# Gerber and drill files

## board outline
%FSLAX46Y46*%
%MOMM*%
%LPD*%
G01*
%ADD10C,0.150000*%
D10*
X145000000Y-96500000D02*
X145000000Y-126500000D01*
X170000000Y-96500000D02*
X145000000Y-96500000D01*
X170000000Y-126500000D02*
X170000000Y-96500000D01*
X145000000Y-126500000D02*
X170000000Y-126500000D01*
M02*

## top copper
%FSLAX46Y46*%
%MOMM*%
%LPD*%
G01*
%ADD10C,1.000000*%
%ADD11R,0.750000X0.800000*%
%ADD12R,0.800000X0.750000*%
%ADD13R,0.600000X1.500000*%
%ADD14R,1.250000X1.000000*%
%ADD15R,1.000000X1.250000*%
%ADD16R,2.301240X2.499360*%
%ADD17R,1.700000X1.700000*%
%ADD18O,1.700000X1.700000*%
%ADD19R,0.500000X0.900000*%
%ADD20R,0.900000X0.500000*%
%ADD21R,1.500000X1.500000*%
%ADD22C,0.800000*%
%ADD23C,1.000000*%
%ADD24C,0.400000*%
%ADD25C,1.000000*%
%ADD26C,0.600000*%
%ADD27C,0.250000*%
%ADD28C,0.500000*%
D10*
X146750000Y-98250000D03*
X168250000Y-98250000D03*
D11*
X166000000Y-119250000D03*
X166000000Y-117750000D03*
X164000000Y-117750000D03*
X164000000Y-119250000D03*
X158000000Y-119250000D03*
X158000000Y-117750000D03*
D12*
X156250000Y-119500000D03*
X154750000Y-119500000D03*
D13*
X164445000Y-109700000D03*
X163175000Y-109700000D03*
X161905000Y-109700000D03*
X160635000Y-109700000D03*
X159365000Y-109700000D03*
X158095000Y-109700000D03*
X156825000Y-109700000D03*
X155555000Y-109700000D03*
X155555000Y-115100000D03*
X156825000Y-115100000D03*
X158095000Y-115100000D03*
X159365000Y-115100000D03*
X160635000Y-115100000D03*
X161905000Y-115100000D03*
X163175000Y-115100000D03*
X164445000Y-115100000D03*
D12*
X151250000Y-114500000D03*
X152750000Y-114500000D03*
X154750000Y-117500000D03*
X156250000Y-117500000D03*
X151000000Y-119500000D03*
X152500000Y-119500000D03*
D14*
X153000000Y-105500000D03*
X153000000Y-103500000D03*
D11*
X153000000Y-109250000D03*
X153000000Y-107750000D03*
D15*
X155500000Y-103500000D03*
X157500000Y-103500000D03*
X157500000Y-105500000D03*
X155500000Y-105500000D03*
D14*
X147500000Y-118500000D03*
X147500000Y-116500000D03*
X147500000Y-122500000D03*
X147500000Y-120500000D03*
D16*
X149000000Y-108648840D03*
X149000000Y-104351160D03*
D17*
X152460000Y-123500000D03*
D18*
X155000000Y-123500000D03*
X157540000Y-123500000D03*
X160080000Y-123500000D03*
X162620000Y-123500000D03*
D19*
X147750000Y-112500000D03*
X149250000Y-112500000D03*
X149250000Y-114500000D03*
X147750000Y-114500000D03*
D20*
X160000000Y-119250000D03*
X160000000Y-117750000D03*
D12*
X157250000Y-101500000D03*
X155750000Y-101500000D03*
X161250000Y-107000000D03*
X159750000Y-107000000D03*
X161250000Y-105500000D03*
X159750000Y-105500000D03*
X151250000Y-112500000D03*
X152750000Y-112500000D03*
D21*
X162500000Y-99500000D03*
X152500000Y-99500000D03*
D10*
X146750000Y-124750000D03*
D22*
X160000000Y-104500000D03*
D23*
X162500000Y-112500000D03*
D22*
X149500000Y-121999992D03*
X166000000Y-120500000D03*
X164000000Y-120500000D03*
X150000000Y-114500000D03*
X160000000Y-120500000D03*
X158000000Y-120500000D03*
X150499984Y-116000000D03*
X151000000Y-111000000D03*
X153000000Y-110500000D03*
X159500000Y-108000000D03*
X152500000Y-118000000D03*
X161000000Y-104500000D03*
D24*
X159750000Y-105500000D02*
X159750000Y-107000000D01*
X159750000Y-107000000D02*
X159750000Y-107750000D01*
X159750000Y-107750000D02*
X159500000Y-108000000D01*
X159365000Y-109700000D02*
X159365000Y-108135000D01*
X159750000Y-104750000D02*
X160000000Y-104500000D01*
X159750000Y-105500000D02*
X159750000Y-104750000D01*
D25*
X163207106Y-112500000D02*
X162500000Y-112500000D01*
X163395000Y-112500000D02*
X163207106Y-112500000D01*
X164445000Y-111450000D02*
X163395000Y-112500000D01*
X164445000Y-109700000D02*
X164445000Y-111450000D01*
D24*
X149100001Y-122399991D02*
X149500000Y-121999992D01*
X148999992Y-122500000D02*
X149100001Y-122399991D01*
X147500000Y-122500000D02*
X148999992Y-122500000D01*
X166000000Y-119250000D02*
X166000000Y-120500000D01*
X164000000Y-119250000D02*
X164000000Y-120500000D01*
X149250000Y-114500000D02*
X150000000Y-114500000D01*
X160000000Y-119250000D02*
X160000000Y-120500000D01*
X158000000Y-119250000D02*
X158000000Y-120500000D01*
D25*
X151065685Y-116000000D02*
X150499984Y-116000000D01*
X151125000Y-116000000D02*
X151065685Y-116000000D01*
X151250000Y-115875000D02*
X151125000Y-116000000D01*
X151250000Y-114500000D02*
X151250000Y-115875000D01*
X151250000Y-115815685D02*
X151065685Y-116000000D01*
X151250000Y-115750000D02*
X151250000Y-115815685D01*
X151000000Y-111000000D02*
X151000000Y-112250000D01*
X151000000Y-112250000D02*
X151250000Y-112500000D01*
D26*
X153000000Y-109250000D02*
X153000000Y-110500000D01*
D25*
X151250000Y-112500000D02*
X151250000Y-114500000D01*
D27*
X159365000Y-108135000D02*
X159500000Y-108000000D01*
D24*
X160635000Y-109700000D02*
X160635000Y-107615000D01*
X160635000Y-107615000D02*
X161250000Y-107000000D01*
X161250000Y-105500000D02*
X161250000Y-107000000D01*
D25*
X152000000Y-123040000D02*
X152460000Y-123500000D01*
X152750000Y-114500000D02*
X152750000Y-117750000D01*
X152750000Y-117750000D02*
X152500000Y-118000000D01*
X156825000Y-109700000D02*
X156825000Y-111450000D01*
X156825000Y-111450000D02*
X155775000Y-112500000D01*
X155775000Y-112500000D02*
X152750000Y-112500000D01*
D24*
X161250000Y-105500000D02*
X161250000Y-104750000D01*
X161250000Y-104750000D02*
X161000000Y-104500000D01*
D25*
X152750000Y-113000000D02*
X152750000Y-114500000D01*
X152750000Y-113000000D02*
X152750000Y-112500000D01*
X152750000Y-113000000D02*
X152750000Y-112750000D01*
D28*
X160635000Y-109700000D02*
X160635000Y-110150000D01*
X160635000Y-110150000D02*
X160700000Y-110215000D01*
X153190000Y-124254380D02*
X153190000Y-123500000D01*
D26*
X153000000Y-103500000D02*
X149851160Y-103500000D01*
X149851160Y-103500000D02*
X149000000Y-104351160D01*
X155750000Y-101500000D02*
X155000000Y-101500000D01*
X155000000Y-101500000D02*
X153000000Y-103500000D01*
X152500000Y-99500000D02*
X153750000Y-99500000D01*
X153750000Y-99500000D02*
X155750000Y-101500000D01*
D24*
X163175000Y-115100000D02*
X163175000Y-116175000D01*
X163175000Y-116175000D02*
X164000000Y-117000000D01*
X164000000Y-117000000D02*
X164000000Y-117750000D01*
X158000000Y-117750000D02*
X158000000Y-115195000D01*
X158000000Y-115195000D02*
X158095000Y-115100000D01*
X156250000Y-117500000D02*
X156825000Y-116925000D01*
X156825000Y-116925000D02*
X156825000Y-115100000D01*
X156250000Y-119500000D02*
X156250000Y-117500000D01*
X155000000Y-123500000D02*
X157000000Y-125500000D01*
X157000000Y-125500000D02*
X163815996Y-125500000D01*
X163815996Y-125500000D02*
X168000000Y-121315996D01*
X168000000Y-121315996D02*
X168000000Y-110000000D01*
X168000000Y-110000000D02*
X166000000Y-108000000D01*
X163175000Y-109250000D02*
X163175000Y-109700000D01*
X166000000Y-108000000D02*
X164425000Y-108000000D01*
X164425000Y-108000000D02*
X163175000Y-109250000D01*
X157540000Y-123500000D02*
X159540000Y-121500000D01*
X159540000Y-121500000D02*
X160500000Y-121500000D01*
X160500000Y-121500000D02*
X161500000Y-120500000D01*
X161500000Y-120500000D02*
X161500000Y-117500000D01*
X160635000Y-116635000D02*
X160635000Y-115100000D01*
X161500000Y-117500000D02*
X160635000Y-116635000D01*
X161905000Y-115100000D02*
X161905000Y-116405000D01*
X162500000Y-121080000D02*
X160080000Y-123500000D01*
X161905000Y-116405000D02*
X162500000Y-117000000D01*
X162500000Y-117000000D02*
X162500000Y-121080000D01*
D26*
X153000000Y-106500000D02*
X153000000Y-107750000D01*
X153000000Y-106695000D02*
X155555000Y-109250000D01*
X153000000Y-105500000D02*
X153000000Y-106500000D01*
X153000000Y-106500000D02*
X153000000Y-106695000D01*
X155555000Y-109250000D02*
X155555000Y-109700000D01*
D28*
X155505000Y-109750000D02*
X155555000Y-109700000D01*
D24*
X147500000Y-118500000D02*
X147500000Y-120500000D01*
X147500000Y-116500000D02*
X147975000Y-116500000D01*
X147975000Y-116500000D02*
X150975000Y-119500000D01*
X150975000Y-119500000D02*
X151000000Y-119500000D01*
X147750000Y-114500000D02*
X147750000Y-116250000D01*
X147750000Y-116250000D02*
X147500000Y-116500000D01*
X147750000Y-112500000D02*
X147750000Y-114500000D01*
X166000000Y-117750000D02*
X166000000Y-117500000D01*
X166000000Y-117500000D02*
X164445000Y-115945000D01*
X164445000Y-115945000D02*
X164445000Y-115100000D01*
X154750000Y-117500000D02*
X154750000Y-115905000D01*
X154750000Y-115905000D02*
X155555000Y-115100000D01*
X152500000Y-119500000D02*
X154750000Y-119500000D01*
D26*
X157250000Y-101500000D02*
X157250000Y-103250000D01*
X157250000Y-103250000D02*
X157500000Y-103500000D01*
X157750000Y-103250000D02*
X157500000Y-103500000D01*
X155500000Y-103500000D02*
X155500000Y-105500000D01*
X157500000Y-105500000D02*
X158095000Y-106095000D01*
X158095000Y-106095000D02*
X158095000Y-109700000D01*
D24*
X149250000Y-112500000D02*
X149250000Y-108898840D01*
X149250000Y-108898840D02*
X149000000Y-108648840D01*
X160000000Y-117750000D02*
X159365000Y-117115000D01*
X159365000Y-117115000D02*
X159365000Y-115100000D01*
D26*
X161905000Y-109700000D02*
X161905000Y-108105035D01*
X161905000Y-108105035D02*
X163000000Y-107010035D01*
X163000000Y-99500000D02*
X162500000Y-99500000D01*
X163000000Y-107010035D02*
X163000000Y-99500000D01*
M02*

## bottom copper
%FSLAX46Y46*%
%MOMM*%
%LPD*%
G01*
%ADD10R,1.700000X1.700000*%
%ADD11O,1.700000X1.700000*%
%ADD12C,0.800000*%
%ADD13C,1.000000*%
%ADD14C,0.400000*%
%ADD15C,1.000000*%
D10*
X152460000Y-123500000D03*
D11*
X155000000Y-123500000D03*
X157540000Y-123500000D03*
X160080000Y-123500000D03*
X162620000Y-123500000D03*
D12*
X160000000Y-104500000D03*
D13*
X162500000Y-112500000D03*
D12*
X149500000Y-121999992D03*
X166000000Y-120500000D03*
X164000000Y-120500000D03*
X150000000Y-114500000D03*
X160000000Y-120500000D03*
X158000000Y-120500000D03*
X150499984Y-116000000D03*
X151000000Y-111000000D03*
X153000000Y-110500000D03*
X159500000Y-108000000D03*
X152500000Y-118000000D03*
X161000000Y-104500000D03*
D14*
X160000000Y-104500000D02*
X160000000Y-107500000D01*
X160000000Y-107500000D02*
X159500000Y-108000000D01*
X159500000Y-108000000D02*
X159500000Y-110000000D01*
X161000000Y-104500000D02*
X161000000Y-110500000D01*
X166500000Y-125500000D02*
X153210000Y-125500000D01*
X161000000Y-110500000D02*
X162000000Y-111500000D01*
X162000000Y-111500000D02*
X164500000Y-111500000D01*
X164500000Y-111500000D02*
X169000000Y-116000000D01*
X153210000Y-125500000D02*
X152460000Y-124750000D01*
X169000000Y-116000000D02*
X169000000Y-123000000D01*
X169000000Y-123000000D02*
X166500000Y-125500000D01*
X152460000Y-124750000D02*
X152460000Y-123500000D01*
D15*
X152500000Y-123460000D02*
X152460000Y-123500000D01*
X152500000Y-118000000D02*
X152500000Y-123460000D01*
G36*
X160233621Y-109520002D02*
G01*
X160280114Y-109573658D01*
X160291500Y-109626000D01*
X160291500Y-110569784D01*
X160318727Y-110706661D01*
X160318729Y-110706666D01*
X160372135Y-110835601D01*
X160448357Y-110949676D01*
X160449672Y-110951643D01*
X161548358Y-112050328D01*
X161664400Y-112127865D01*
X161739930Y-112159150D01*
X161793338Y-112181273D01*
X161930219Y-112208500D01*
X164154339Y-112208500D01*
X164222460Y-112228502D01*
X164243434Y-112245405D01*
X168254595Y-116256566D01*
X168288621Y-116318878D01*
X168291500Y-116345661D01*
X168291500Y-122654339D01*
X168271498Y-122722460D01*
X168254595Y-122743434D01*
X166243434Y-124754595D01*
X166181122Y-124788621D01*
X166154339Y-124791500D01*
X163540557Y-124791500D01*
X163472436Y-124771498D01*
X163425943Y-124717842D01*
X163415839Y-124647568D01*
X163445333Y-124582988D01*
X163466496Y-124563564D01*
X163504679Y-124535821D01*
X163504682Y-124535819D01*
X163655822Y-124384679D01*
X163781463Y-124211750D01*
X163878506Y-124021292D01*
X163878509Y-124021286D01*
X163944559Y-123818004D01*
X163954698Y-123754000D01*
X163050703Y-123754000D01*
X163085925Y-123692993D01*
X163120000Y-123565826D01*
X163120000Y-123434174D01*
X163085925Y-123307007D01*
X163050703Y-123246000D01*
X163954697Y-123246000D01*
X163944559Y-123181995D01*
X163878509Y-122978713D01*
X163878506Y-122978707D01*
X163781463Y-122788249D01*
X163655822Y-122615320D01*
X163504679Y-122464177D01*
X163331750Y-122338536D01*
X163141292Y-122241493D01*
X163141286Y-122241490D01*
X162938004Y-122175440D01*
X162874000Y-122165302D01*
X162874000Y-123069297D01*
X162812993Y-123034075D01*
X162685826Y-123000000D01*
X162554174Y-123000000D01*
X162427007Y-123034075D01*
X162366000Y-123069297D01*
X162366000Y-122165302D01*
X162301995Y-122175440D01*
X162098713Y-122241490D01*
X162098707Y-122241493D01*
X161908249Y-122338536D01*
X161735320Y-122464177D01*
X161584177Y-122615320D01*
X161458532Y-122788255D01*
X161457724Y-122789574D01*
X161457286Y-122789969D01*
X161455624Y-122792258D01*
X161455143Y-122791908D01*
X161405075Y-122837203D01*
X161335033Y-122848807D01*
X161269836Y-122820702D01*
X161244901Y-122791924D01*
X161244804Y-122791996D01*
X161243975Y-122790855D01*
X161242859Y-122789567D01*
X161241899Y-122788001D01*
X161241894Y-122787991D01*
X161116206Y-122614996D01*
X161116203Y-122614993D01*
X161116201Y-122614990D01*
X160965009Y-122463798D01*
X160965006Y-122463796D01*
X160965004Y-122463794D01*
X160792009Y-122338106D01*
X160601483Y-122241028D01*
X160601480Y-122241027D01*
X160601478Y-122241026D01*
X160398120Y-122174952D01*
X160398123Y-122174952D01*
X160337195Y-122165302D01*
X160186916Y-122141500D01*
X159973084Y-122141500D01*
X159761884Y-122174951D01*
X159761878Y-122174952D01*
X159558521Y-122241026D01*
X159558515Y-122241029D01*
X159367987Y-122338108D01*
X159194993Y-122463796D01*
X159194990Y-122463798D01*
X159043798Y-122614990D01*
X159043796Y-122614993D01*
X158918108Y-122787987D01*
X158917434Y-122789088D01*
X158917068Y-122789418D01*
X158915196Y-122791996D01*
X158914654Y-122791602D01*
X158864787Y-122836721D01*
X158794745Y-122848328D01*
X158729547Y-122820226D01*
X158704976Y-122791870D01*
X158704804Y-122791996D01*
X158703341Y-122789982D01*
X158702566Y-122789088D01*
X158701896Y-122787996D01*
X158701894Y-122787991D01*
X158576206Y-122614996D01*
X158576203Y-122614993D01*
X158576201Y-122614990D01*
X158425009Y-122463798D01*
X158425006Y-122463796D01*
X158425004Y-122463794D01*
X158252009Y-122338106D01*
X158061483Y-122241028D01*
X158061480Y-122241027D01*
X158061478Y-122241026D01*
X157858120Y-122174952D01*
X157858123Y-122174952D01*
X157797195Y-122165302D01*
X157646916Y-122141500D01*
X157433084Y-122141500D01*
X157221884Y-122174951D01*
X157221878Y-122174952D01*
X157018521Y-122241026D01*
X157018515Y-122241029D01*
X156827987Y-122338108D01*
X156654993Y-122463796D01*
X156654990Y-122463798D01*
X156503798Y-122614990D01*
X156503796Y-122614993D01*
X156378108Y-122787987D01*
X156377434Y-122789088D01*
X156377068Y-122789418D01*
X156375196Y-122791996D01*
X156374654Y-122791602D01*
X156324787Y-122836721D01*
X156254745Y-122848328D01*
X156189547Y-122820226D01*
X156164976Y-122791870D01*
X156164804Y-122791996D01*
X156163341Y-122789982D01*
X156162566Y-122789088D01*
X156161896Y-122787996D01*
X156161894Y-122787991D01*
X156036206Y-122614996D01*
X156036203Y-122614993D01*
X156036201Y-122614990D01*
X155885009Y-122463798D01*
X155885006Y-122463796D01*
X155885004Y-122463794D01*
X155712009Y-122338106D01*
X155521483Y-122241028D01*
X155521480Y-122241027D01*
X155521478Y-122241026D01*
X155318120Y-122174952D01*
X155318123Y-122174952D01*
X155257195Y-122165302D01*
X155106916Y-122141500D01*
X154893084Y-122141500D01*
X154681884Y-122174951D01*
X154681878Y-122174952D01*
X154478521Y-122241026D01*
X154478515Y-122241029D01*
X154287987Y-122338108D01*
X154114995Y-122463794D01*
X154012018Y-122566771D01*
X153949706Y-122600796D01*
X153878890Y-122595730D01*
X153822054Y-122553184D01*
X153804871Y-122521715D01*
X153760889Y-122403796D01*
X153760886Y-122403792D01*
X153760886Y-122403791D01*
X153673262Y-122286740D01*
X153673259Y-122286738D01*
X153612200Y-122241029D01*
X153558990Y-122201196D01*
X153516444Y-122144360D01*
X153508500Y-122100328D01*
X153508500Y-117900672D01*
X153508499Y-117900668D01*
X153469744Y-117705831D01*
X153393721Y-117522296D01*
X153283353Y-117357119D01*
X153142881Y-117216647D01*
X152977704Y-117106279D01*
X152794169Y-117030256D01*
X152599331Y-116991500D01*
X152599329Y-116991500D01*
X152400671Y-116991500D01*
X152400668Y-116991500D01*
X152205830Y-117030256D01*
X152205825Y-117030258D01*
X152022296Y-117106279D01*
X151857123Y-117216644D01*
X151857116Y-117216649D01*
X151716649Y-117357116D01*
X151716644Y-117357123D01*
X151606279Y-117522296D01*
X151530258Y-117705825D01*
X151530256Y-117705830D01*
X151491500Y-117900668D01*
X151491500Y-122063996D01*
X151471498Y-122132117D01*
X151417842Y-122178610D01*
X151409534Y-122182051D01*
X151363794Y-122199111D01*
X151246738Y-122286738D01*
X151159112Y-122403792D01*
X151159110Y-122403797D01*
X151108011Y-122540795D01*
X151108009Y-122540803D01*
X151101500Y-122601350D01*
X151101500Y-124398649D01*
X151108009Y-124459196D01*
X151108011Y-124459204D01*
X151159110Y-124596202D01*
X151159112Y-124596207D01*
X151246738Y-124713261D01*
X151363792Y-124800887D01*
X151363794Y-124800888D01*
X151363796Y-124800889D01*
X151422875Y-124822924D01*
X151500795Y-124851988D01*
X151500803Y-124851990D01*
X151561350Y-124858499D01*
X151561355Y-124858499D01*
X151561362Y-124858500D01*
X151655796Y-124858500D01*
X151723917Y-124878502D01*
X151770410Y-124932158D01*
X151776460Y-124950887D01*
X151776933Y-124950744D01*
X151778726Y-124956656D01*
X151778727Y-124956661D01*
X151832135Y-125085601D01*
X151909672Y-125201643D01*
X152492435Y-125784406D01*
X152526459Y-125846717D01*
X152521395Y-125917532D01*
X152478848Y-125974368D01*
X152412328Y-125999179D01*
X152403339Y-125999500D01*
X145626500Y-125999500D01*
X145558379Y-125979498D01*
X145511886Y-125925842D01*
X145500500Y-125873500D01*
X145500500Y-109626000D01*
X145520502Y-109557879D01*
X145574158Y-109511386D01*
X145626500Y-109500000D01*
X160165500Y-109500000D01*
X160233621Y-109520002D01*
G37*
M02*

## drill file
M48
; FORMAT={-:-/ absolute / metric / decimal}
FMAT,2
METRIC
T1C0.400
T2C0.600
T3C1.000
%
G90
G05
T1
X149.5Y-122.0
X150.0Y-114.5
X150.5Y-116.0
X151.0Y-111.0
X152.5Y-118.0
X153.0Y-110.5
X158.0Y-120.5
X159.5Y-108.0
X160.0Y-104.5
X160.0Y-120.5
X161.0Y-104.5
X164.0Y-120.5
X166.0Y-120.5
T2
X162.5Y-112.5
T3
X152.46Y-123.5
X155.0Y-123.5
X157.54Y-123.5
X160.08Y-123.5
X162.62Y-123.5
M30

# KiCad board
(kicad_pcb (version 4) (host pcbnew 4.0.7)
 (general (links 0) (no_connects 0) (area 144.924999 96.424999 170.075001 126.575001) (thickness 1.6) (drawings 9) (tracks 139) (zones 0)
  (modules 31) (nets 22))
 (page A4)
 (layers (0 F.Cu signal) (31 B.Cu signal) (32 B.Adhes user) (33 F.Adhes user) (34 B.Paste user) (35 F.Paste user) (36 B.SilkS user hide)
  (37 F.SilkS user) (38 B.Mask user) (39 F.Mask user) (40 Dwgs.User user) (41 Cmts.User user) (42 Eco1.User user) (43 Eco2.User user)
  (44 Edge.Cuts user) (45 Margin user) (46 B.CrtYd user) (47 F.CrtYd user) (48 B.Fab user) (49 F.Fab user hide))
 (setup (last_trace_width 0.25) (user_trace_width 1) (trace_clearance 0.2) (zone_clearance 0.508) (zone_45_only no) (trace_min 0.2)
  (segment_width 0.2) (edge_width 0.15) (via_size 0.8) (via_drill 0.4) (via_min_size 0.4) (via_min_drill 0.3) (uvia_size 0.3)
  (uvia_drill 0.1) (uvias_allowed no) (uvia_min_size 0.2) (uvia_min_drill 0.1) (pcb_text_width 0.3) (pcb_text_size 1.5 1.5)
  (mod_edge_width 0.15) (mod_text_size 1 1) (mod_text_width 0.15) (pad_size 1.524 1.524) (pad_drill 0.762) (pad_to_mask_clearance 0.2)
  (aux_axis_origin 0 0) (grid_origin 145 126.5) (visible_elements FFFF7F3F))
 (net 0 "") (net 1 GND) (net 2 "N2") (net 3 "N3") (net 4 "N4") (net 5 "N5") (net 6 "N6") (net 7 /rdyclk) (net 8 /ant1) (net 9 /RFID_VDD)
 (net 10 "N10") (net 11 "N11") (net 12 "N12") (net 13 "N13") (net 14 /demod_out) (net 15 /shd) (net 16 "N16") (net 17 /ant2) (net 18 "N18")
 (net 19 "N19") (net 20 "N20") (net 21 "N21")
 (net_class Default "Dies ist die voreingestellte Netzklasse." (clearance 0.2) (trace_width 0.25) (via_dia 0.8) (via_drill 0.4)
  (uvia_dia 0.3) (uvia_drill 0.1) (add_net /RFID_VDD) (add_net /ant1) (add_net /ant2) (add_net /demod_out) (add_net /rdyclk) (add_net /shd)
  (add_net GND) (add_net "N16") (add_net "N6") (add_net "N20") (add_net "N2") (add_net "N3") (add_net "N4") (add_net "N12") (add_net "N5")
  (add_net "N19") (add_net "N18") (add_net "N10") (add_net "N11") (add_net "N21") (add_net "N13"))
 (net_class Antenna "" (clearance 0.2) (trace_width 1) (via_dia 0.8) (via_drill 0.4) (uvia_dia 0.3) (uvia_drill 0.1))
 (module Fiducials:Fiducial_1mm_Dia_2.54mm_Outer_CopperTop (layer F.Cu) (at 146.75 98.25)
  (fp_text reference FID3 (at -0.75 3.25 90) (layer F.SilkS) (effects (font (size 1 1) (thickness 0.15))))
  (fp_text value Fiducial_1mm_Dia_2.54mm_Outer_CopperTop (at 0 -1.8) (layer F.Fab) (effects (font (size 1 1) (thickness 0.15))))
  (pad ~ smd circle (at 0 0) (size 1 1) (layers F.Cu F.Mask) (solder_mask_margin 0.77) (clearance 0.77)))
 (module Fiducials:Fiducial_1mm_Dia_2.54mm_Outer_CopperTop (layer F.Cu) (at 168.25 98.25)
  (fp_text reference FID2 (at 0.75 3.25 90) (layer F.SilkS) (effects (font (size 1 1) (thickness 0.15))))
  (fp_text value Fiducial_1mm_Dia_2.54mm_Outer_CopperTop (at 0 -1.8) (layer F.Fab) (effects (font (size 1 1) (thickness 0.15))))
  (pad ~ smd circle (at 0 0) (size 1 1) (layers F.Cu F.Mask) (solder_mask_margin 0.77) (clearance 0.77)))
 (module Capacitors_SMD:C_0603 (layer F.Cu) (at 166 118.5 90)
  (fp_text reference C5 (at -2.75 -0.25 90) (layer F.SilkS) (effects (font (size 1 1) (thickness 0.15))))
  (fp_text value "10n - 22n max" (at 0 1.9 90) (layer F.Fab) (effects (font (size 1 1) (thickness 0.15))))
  (pad 1 smd rect (at -0.75 0 90) (size 0.8 0.75) (layers F.Cu F.Paste F.Mask) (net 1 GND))
  (pad 2 smd rect (at 0.75 0 90) (size 0.8 0.75) (layers F.Cu F.Paste F.Mask) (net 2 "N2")))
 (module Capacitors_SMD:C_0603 (layer F.Cu) (at 164 118.5 90)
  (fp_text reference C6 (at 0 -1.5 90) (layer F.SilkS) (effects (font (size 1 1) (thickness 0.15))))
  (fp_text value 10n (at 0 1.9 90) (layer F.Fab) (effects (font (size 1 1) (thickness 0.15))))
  (pad 2 smd rect (at 0.75 0 90) (size 0.8 0.75) (layers F.Cu F.Paste F.Mask) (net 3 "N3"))
  (pad 1 smd rect (at -0.75 0 90) (size 0.8 0.75) (layers F.Cu F.Paste F.Mask) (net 1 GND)))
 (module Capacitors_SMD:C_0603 (layer F.Cu) (at 158 118.5 90)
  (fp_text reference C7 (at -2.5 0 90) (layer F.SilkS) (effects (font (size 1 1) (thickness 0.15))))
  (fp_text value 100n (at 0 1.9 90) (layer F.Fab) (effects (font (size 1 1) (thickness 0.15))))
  (pad 1 smd rect (at -0.75 0 90) (size 0.8 0.75) (layers F.Cu F.Paste F.Mask) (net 1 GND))
  (pad 2 smd rect (at 0.75 0 90) (size 0.8 0.75) (layers F.Cu F.Paste F.Mask) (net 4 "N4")))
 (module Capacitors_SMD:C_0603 (layer F.Cu) (at 155.5 119.5)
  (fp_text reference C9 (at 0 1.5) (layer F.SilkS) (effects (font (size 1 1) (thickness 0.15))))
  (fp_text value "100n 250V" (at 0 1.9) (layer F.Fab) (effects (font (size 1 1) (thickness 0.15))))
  (pad 2 smd rect (at 0.75 0) (size 0.8 0.75) (layers F.Cu F.Paste F.Mask) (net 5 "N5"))
  (pad 1 smd rect (at -0.75 0) (size 0.8 0.75) (layers F.Cu F.Paste F.Mask) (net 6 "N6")))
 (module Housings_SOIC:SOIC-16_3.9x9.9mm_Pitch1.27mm (layer F.Cu) (at 160 112.4 270)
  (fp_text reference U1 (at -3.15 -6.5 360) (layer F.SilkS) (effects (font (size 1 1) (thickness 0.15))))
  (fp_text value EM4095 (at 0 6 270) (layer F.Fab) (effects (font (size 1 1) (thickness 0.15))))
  (pad 1 smd rect (at -2.7 -4.445 270) (size 1.5 0.6) (layers F.Cu F.Paste F.Mask) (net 1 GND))
  (pad 2 smd rect (at -2.7 -3.175 270) (size 1.5 0.6) (layers F.Cu F.Paste F.Mask) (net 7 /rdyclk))
  (pad 3 smd rect (at -2.7 -1.905 270) (size 1.5 0.6) (layers F.Cu F.Paste F.Mask) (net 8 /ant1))
  (pad 4 smd rect (at -2.7 -0.635 270) (size 1.5 0.6) (layers F.Cu F.Paste F.Mask) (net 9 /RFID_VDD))
  (pad 5 smd rect (at -2.7 0.635 270) (size 1.5 0.6) (layers F.Cu F.Paste F.Mask) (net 1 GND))
  (pad 6 smd rect (at -2.7 1.905 270) (size 1.5 0.6) (layers F.Cu F.Paste F.Mask) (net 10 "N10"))
  (pad 7 smd rect (at -2.7 3.175 270) (size 1.5 0.6) (layers F.Cu F.Paste F.Mask) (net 9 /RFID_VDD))
  (pad 8 smd rect (at -2.7 4.445 270) (size 1.5 0.6) (layers F.Cu F.Paste F.Mask) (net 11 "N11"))
  (pad 9 smd rect (at 2.7 4.445 270) (size 1.5 0.6) (layers F.Cu F.Paste F.Mask) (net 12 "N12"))
  (pad 10 smd rect (at 2.7 3.175 270) (size 1.5 0.6) (layers F.Cu F.Paste F.Mask) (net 5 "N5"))
  (pad 11 smd rect (at 2.7 1.905 270) (size 1.5 0.6) (layers F.Cu F.Paste F.Mask) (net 4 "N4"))
  (pad 12 smd rect (at 2.7 0.635 270) (size 1.5 0.6) (layers F.Cu F.Paste F.Mask) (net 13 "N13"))
  (pad 13 smd rect (at 2.7 -0.635 270) (size 1.5 0.6) (layers F.Cu F.Paste F.Mask) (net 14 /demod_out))
  (pad 14 smd rect (at 2.7 -1.905 270) (size 1.5 0.6) (layers F.Cu F.Paste F.Mask) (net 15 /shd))
  (pad 15 smd rect (at 2.7 -3.175 270) (size 1.5 0.6) (layers F.Cu F.Paste F.Mask) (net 3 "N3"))
  (pad 16 smd rect (at 2.7 -4.445 270) (size 1.5 0.6) (layers F.Cu F.Paste F.Mask) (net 2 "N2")))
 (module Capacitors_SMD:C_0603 (layer F.Cu) (at 152 114.5)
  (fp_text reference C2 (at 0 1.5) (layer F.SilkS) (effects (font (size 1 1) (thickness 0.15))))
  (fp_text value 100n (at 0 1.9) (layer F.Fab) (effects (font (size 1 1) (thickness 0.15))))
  (pad 1 smd rect (at -0.75 0) (size 0.8 0.75) (layers F.Cu F.Paste F.Mask) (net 1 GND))
  (pad 2 smd rect (at 0.75 0) (size 0.8 0.75) (layers F.Cu F.Paste F.Mask) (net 9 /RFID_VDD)))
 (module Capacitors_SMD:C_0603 (layer F.Cu) (at 155.5 117.5)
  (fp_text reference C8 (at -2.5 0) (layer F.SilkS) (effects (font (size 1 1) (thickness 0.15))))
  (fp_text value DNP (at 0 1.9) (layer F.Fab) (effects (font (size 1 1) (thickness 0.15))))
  (pad 1 smd rect (at -0.75 0) (size 0.8 0.75) (layers F.Cu F.Paste F.Mask) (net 12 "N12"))
  (pad 2 smd rect (at 0.75 0) (size 0.8 0.75) (layers F.Cu F.Paste F.Mask) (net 5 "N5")))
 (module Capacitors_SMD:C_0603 (layer F.Cu) (at 151.75 119.5)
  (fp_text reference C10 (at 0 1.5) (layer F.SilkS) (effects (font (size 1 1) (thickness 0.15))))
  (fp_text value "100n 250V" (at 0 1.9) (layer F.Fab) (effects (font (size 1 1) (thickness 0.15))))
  (pad 1 smd rect (at -0.75 0) (size 0.8 0.75) (layers F.Cu F.Paste F.Mask) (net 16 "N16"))
  (pad 2 smd rect (at 0.75 0) (size 0.8 0.75) (layers F.Cu F.Paste F.Mask) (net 6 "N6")))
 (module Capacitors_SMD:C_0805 (layer F.Cu) (at 153 104.5 90)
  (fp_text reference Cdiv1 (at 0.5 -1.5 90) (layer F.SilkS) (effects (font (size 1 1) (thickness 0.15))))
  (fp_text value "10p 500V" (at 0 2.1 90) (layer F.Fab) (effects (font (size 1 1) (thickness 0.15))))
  (pad 1 smd rect (at -1 0 90) (size 1 1.25) (layers F.Cu F.Paste F.Mask) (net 11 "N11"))
  (pad 2 smd rect (at 1 0 90) (size 1 1.25) (layers F.Cu F.Paste F.Mask) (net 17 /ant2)))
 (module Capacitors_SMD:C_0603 (layer F.Cu) (at 153 108.5 90)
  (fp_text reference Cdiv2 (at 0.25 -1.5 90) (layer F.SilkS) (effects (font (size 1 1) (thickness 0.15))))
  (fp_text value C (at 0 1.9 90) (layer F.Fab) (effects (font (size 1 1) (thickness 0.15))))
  (pad 1 smd rect (at -0.75 0 90) (size 0.8 0.75) (layers F.Cu F.Paste F.Mask) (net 1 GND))
  (pad 2 smd rect (at 0.75 0 90) (size 0.8 0.75) (layers F.Cu F.Paste F.Mask) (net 11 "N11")))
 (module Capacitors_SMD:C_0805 (layer F.Cu) (at 156.5 103.5)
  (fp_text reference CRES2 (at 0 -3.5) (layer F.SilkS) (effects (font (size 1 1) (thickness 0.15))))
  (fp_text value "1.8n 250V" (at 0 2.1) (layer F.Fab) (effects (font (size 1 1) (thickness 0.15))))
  (pad 1 smd rect (at -1 0) (size 1 1.25) (layers F.Cu F.Paste F.Mask) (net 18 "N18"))
  (pad 2 smd rect (at 1 0) (size 1 1.25) (layers F.Cu F.Paste F.Mask) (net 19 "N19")))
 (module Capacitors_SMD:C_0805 (layer F.Cu) (at 156.5 105.5 180)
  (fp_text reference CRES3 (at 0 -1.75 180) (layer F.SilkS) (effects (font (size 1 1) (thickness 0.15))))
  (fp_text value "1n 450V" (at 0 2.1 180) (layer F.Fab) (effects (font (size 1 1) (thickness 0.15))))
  (pad 1 smd rect (at -1 0 180) (size 1 1.25) (layers F.Cu F.Paste F.Mask) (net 10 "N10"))
  (pad 2 smd rect (at 1 0 180) (size 1 1.25) (layers F.Cu F.Paste F.Mask) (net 18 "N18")))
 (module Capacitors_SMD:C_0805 (layer F.Cu) (at 147.5 117.5 90)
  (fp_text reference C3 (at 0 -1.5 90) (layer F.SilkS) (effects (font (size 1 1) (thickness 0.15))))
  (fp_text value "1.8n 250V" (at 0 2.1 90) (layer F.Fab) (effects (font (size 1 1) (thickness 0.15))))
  (pad 1 smd rect (at -1 0 90) (size 1 1.25) (layers F.Cu F.Paste F.Mask) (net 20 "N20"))
  (pad 2 smd rect (at 1 0 90) (size 1 1.25) (layers F.Cu F.Paste F.Mask) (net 16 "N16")))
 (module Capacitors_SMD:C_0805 (layer F.Cu) (at 147.5 121.5 90)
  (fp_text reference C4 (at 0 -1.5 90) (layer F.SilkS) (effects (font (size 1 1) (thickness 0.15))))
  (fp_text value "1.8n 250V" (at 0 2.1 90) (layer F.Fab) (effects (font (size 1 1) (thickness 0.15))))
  (pad 1 smd rect (at -1 0 90) (size 1 1.25) (layers F.Cu F.Paste F.Mask) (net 1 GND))
  (pad 2 smd rect (at 1 0 90) (size 1 1.25) (layers F.Cu F.Paste F.Mask) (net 20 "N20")))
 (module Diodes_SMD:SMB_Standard (layer F.Cu) (at 149 106.5 90)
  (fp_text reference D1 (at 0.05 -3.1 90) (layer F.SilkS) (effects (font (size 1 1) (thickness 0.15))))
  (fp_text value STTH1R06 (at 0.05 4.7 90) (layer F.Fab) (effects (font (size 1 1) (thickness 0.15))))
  (pad 1 smd rect (at -2.14884 0 90) (size 2.49936 2.30124) (layers F.Cu F.Paste F.Mask) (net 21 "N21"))
  (pad 2 smd rect (at 2.14884 0 90) (size 2.49936 2.30124) (layers F.Cu F.Paste F.Mask) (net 17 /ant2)))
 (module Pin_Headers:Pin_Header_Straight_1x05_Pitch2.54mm (layer F.Cu) (at 152.46 123.5 90)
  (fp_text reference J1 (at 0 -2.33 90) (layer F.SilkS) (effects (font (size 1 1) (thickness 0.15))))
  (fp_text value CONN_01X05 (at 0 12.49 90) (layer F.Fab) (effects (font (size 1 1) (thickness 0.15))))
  (pad 1 thru_hole rect (at 0 0 90) (size 1.7 1.7) (drill 1) (layers *.Cu *.Mask) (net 9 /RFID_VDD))
  (pad 2 thru_hole oval (at 0 2.54 90) (size 1.7 1.7) (drill 1) (layers *.Cu *.Mask) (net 7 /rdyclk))
  (pad 3 thru_hole oval (at 0 5.08 90) (size 1.7 1.7) (drill 1) (layers *.Cu *.Mask) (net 14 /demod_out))
  (pad 4 thru_hole oval (at 0 7.62 90) (size 1.7 1.7) (drill 1) (layers *.Cu *.Mask) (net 15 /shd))
  (pad 5 thru_hole oval (at 0 10.16 90) (size 1.7 1.7) (drill 1) (layers *.Cu *.Mask) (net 1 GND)))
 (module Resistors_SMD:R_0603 (layer F.Cu) (at 148.5 112.5)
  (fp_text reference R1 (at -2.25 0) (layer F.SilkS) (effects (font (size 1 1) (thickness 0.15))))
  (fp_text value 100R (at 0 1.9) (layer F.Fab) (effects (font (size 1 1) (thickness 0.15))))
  (pad 1 smd rect (at -0.75 0) (size 0.5 0.9) (layers F.Cu F.Paste F.Mask) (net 16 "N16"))
  (pad 2 smd rect (at 0.75 0) (size 0.5 0.9) (layers F.Cu F.Paste F.Mask) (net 21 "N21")))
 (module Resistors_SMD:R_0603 (layer F.Cu) (at 148.5 114.5 180)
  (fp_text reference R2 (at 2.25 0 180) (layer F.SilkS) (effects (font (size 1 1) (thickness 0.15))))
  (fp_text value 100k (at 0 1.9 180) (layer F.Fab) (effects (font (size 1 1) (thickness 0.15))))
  (pad 1 smd rect (at -0.75 0 180) (size 0.5 0.9) (layers F.Cu F.Paste F.Mask) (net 1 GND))
  (pad 2 smd rect (at 0.75 0 180) (size 0.5 0.9) (layers F.Cu F.Paste F.Mask) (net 16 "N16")))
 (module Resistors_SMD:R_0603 (layer F.Cu) (at 160 118.5 90)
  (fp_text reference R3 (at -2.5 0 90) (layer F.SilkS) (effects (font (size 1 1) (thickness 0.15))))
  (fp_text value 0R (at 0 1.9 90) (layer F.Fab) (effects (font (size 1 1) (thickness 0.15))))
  (pad 1 smd rect (at -0.75 0 90) (size 0.5 0.9) (layers F.Cu F.Paste F.Mask) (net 1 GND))
  (pad 2 smd rect (at 0.75 0 90) (size 0.5 0.9) (layers F.Cu F.Paste F.Mask) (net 13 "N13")))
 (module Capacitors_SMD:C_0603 (layer F.Cu) (at 156.5 101.5 180)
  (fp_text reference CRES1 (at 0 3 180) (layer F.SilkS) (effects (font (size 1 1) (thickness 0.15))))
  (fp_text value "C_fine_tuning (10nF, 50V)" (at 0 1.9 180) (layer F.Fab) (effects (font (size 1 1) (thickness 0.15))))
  (pad 1 smd rect (at -0.75 0 180) (size 0.8 0.75) (layers F.Cu F.Paste F.Mask) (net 19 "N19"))
  (pad 2 smd rect (at 0.75 0 180) (size 0.8 0.75) (layers F.Cu F.Paste F.Mask) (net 17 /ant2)))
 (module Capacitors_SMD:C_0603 (layer F.Cu) (at 160.5 107 180)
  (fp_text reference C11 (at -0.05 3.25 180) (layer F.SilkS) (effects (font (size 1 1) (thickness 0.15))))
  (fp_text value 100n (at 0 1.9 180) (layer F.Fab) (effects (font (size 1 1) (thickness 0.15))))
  (pad 1 smd rect (at -0.75 0 180) (size 0.8 0.75) (layers F.Cu F.Paste F.Mask) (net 9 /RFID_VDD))
  (pad 2 smd rect (at 0.75 0 180) (size 0.8 0.75) (layers F.Cu F.Paste F.Mask) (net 1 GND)))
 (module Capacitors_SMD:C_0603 (layer F.Cu) (at 160.5 105.5 180)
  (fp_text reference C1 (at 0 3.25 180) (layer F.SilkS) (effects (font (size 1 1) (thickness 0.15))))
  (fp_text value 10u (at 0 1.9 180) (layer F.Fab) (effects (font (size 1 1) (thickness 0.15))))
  (pad 1 smd rect (at -0.75 0 180) (size 0.8 0.75) (layers F.Cu F.Paste F.Mask) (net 9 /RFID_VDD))
  (pad 2 smd rect (at 0.75 0 180) (size 0.8 0.75) (layers F.Cu F.Paste F.Mask) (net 1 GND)))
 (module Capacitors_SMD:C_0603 (layer F.Cu) (at 152 112.5)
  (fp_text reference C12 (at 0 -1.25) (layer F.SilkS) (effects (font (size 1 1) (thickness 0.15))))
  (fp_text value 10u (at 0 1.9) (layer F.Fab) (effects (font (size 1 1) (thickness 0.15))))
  (pad 1 smd rect (at -0.75 0) (size 0.8 0.75) (layers F.Cu F.Paste F.Mask) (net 1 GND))
  (pad 2 smd rect (at 0.75 0) (size 0.8 0.75) (layers F.Cu F.Paste F.Mask) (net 9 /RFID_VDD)))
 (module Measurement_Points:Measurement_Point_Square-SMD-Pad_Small (layer F.Cu) (at 162.5 99.5)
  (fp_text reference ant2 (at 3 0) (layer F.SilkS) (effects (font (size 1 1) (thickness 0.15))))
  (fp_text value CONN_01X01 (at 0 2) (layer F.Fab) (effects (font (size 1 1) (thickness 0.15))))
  (pad 1 smd rect (at 0 0) (size 1.5 1.5) (layers F.Cu F.Mask) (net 8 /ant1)))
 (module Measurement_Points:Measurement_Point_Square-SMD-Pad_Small (layer F.Cu) (at 152.5 99.5)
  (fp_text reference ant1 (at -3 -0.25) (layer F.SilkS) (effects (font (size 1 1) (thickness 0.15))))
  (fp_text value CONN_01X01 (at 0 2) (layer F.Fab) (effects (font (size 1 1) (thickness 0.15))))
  (pad 1 smd rect (at 0 0) (size 1.5 1.5) (layers F.Cu F.Mask) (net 17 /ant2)))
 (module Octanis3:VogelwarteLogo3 (layer B.Cu) (at 158 116.5 180)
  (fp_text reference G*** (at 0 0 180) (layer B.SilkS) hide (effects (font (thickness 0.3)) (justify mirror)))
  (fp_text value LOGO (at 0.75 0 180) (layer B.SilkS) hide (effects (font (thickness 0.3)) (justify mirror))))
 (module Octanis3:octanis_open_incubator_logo (layer B.Cu) (at 158 104.5 180)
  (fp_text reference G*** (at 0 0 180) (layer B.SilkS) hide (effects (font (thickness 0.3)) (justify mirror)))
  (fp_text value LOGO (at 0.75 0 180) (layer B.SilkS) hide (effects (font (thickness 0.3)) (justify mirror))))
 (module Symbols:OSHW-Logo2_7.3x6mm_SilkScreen (layer F.Cu) (at 165.95 105.15)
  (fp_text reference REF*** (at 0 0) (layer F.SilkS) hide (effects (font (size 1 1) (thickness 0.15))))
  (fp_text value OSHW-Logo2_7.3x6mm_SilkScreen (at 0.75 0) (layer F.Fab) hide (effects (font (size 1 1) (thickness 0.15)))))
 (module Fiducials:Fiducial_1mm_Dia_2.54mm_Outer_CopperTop (layer F.Cu) (at 146.75 124.75)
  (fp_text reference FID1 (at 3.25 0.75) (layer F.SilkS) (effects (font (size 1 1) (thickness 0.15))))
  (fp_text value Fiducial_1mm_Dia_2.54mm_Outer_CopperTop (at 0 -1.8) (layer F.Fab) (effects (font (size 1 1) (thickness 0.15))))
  (pad ~ smd circle (at 0 0) (size 1 1) (layers F.Cu F.Mask) (solder_mask_margin 0.77) (clearance 0.77)))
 (gr_line (start 145 96.5) (end 145 126.5) (layer Edge.Cuts) (width 0.15))
 (gr_line (start 170 96.5) (end 145 96.5) (layer Edge.Cuts) (width 0.15))
 (gr_line (start 170 126.5) (end 170 96.5) (layer Edge.Cuts) (width 0.15))
 (gr_line (start 145 126.5) (end 170 126.5) (layer Edge.Cuts) (width 0.15))
 (segment (start 159.75 105.5) (end 159.75 107) (width 0.4) (layer F.Cu) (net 1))
 (segment (start 159.75 107) (end 159.75 107.75) (width 0.4) (layer F.Cu) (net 1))
 (segment (start 159.75 107.75) (end 159.5 108) (width 0.4) (layer F.Cu) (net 1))
 (segment (start 159.365 109.7) (end 159.365 108.135) (width 0.4) (layer F.Cu) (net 1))
 (segment (start 159.75 104.75) (end 160 104.5) (width 0.4) (layer F.Cu) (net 1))
 (segment (start 159.75 105.5) (end 159.75 104.75) (width 0.4) (layer F.Cu) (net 1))
 (segment (start 160 104.5) (end 160 107.5) (width 0.4) (layer B.Cu) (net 1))
 (segment (start 160 107.5) (end 159.5 108) (width 0.4) (layer B.Cu) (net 1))
 (via (at 160 104.5) (size 0.8) (drill 0.4) (layers F.Cu B.Cu) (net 1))
 (segment (start 159.5 108) (end 159.5 110) (width 0.4) (layer B.Cu) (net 1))
 (segment (start 163.207106 112.5) (end 162.5 112.5) (width 1) (layer F.Cu) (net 1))
 (segment (start 163.395 112.5) (end 163.207106 112.5) (width 1) (layer F.Cu) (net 1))
 (segment (start 164.445 111.45) (end 163.395 112.5) (width 1) (layer F.Cu) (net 1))
 (segment (start 164.445 109.7) (end 164.445 111.45) (width 1) (layer F.Cu) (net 1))
 (via (at 162.5 112.5) (size 1) (drill 0.6) (layers F.Cu B.Cu) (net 1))
 (segment (start 149.100001 122.399991) (end 149.5 121.999992) (width 0.4) (layer F.Cu) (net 1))
 (segment (start 148.999992 122.5) (end 149.100001 122.399991) (width 0.4) (layer F.Cu) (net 1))
 (segment (start 147.5 122.5) (end 148.999992 122.5) (width 0.4) (layer F.Cu) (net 1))
 (via (at 149.5 121.999992) (size 0.8) (drill 0.4) (layers F.Cu B.Cu) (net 1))
 (segment (start 166 119.25) (end 166 120.5) (width 0.4) (layer F.Cu) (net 1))
 (via (at 166 120.5) (size 0.8) (drill 0.4) (layers F.Cu B.Cu) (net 1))
 (segment (start 164 119.25) (end 164 120.5) (width 0.4) (layer F.Cu) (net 1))
 (via (at 164 120.5) (size 0.8) (drill 0.4) (layers F.Cu B.Cu) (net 1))
 (segment (start 149.25 114.5) (end 150 114.5) (width 0.4) (layer F.Cu) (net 1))
 (via (at 150 114.5) (size 0.8) (drill 0.4) (layers F.Cu B.Cu) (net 1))
 (segment (start 160 119.25) (end 160 120.5) (width 0.4) (layer F.Cu) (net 1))
 (via (at 160 120.5) (size 0.8) (drill 0.4) (layers F.Cu B.Cu) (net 1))
 (segment (start 158 119.25) (end 158 120.5) (width 0.4) (layer F.Cu) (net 1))
 (via (at 158 120.5) (size 0.8) (drill 0.4) (layers F.Cu B.Cu) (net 1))
 (segment (start 151.065685 116) (end 150.499984 116) (width 1) (layer F.Cu) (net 1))
 (via (at 150.499984 116) (size 0.8) (drill 0.4) (layers F.Cu B.Cu) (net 1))
 (segment (start 151.125 116) (end 151.065685 116) (width 1) (layer F.Cu) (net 1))
 (segment (start 151.25 115.875) (end 151.125 116) (width 1) (layer F.Cu) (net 1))
 (segment (start 151.25 114.5) (end 151.25 115.875) (width 1) (layer F.Cu) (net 1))
 (segment (start 151.25 115.815685) (end 151.065685 116) (width 1) (layer F.Cu) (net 1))
 (segment (start 151.25 115.75) (end 151.25 115.815685) (width 1) (layer F.Cu) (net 1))
 (segment (start 151 111) (end 151 112.25) (width 1) (layer F.Cu) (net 1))
 (segment (start 151 112.25) (end 151.25 112.5) (width 1) (layer F.Cu) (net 1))
 (via (at 151 111) (size 0.8) (drill 0.4) (layers F.Cu B.Cu) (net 1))
 (segment (start 153 109.25) (end 153 110.5) (width 0.6) (layer F.Cu) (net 1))
 (via (at 153 110.5) (size 0.8) (drill 0.4) (layers F.Cu B.Cu) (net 1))
 (segment (start 151.25 112.5) (end 151.25 114.5) (width 1) (layer F.Cu) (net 1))
 (via (at 159.5 108) (size 0.8) (drill 0.4) (layers F.Cu B.Cu) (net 1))
 (segment (start 159.365 108.135) (end 159.5 108) (width 0.25) (layer F.Cu) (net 1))
 (segment (start 160.635 109.7) (end 160.635 107.615) (width 0.4) (layer F.Cu) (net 9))
 (segment (start 160.635 107.615) (end 161.25 107) (width 0.4) (layer F.Cu) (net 9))
 (segment (start 161.25 105.5) (end 161.25 107) (width 0.4) (layer F.Cu) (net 9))
 (segment (start 161 104.5) (end 161 110.5) (width 0.4) (layer B.Cu) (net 9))
 (segment (start 166.5 125.5) (end 153.21 125.5) (width 0.4) (layer B.Cu) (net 9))
 (segment (start 161 110.5) (end 162 111.5) (width 0.4) (layer B.Cu) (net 9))
 (segment (start 162 111.5) (end 164.5 111.5) (width 0.4) (layer B.Cu) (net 9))
 (segment (start 164.5 111.5) (end 169 116) (width 0.4) (layer B.Cu) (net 9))
 (segment (start 153.21 125.5) (end 152.46 124.75) (width 0.4) (layer B.Cu) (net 9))
 (segment (start 169 116) (end 169 123) (width 0.4) (layer B.Cu) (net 9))
 (segment (start 169 123) (end 166.5 125.5) (width 0.4) (layer B.Cu) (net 9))
 (segment (start 152.46 124.75) (end 152.46 123.5) (width 0.4) (layer B.Cu) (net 9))
 (segment (start 152.5 123.46) (end 152.46 123.5) (width 1) (layer B.Cu) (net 9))
 (segment (start 152.5 118) (end 152.5 123.46) (width 1) (layer B.Cu) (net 9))
 (segment (start 152 123.04) (end 152.46 123.5) (width 1) (layer F.Cu) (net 9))
 (segment (start 152.75 114.5) (end 152.75 117.75) (width 1) (layer F.Cu) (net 9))
 (segment (start 152.75 117.75) (end 152.5 118) (width 1) (layer F.Cu) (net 9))
 (via (at 152.5 118) (size 0.8) (drill 0.4) (layers F.Cu B.Cu) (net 9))
 (segment (start 156.825 109.7) (end 156.825 111.45) (width 1) (layer F.Cu) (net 9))
 (segment (start 156.825 111.45) (end 155.775 112.5) (width 1) (layer F.Cu) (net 9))
 (segment (start 155.775 112.5) (end 152.75 112.5) (width 1) (layer F.Cu) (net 9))
 (segment (start 161.25 105.5) (end 161.25 104.75) (width 0.4) (layer F.Cu) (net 9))
 (segment (start 161.25 104.75) (end 161 104.5) (width 0.4) (layer F.Cu) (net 9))
 (via (at 161 104.5) (size 0.8) (drill 0.4) (layers F.Cu B.Cu) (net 9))
 (segment (start 152.75 113) (end 152.75 114.5) (width 1) (layer F.Cu) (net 9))
 (segment (start 152.75 113) (end 152.75 112.5) (width 1) (layer F.Cu) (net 9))
 (segment (start 152.75 113) (end 152.75 112.75) (width 1) (layer F.Cu) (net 9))
 (segment (start 160.635 109.7) (end 160.635 110.15) (width 0.5) (layer F.Cu) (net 9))
 (segment (start 160.635 110.15) (end 160.7 110.215) (width 0.5) (layer F.Cu) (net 9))
 (segment (start 153.19 124.25438) (end 153.19 123.5) (width 0.5) (layer F.Cu) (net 9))
 (segment (start 153 103.5) (end 149.85116 103.5) (width 0.6) (layer F.Cu) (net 17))
 (segment (start 149.85116 103.5) (end 149 104.35116) (width 0.6) (layer F.Cu) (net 17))
 (segment (start 155.75 101.5) (end 155 101.5) (width 0.6) (layer F.Cu) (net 17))
 (segment (start 155 101.5) (end 153 103.5) (width 0.6) (layer F.Cu) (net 17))
 (segment (start 152.5 99.5) (end 153.75 99.5) (width 0.6) (layer F.Cu) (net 17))
 (segment (start 153.75 99.5) (end 155.75 101.5) (width 0.6) (layer F.Cu) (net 17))
 (segment (start 163.175 115.1) (end 163.175 116.175) (width 0.4) (layer F.Cu) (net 3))
 (segment (start 163.175 116.175) (end 164 117) (width 0.4) (layer F.Cu) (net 3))
 (segment (start 164 117) (end 164 117.75) (width 0.4) (layer F.Cu) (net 3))
 (segment (start 158 117.75) (end 158 115.195) (width 0.4) (layer F.Cu) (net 4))
 (segment (start 158 115.195) (end 158.095 115.1) (width 0.4) (layer F.Cu) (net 4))
 (segment (start 156.25 117.5) (end 156.825 116.925) (width 0.4) (layer F.Cu) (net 5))
 (segment (start 156.825 116.925) (end 156.825 115.1) (width 0.4) (layer F.Cu) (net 5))
 (segment (start 156.25 119.5) (end 156.25 117.5) (width 0.4) (layer F.Cu) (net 5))
 (segment (start 155 123.5) (end 157 125.5) (width 0.4) (layer F.Cu) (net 7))
 (segment (start 157 125.5) (end 163.815996 125.5) (width 0.4) (layer F.Cu) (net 7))
 (segment (start 163.815996 125.5) (end 168 121.315996) (width 0.4) (layer F.Cu) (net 7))
 (segment (start 168 121.315996) (end 168 110) (width 0.4) (layer F.Cu) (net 7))
 (segment (start 168 110) (end 166 108) (width 0.4) (layer F.Cu) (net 7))
 (segment (start 163.175 109.25) (end 163.175 109.7) (width 0.4) (layer F.Cu) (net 7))
 (segment (start 166 108) (end 164.425 108) (width 0.4) (layer F.Cu) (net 7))
 (segment (start 164.425 108) (end 163.175 109.25) (width 0.4) (layer F.Cu) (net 7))
 (segment (start 157.54 123.5) (end 159.54 121.5) (width 0.4) (layer F.Cu) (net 14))
 (segment (start 159.54 121.5) (end 160.5 121.5) (width 0.4) (layer F.Cu) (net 14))
 (segment (start 160.5 121.5) (end 161.5 120.5) (width 0.4) (layer F.Cu) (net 14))
 (segment (start 161.5 120.5) (end 161.5 117.5) (width 0.4) (layer F.Cu) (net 14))
 (segment (start 160.635 116.635) (end 160.635 115.1) (width 0.4) (layer F.Cu) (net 14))
 (segment (start 161.5 117.5) (end 160.635 116.635) (width 0.4) (layer F.Cu) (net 14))
 (segment (start 161.905 115.1) (end 161.905 116.405) (width 0.4) (layer F.Cu) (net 15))
 (segment (start 162.5 121.08) (end 160.08 123.5) (width 0.4) (layer F.Cu) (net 15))
 (segment (start 161.905 116.405) (end 162.5 117) (width 0.4) (layer F.Cu) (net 15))
 (segment (start 162.5 117) (end 162.5 121.08) (width 0.4) (layer F.Cu) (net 15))
 (segment (start 153 106.5) (end 153 107.75) (width 0.6) (layer F.Cu) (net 11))
 (segment (start 153 106.695) (end 155.555 109.25) (width 0.6) (layer F.Cu) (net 11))
 (segment (start 153 105.5) (end 153 106.5) (width 0.6) (layer F.Cu) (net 11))
 (segment (start 153 106.5) (end 153 106.695) (width 0.6) (layer F.Cu) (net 11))
 (segment (start 155.555 109.25) (end 155.555 109.7) (width 0.6) (layer F.Cu) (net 11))
 (segment (start 155.505 109.75) (end 155.555 109.7) (width 0.5) (layer F.Cu) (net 11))
 (segment (start 147.5 118.5) (end 147.5 120.5) (width 0.4) (layer F.Cu) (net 20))
 (segment (start 147.5 116.5) (end 147.975 116.5) (width 0.4) (layer F.Cu) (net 16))
 (segment (start 147.975 116.5) (end 150.975 119.5) (width 0.4) (layer F.Cu) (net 16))
 (segment (start 150.975 119.5) (end 151 119.5) (width 0.4) (layer F.Cu) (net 16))
 (segment (start 147.75 114.5) (end 147.75 116.25) (width 0.4) (layer F.Cu) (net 16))
 (segment (start 147.75 116.25) (end 147.5 116.5) (width 0.4) (layer F.Cu) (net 16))
 (segment (start 147.75 112.5) (end 147.75 114.5) (width 0.4) (layer F.Cu) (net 16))
 (segment (start 166 117.75) (end 166 117.5) (width 0.4) (layer F.Cu) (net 2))
 (segment (start 166 117.5) (end 164.445 115.945) (width 0.4) (layer F.Cu) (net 2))
 (segment (start 164.445 115.945) (end 164.445 115.1) (width 0.4) (layer F.Cu) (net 2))
 (segment (start 154.75 117.5) (end 154.75 115.905) (width 0.4) (layer F.Cu) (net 12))
 (segment (start 154.75 115.905) (end 155.555 115.1) (width 0.4) (layer F.Cu) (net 12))
 (segment (start 152.5 119.5) (end 154.75 119.5) (width 0.4) (layer F.Cu) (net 6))
 (segment (start 157.25 101.5) (end 157.25 103.25) (width 0.6) (layer F.Cu) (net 19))
 (segment (start 157.25 103.25) (end 157.5 103.5) (width 0.6) (layer F.Cu) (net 19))
 (segment (start 157.75 103.25) (end 157.5 103.5) (width 0.6) (layer F.Cu) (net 19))
 (segment (start 155.5 103.5) (end 155.5 105.5) (width 0.6) (layer F.Cu) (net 18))
 (segment (start 157.5 105.5) (end 158.095 106.095) (width 0.6) (layer F.Cu) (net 10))
 (segment (start 158.095 106.095) (end 158.095 109.7) (width 0.6) (layer F.Cu) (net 10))
 (segment (start 149.25 112.5) (end 149.25 108.89884) (width 0.4) (layer F.Cu) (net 21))
 (segment (start 149.25 108.89884) (end 149 108.64884) (width 0.4) (layer F.Cu) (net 21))
 (segment (start 160 117.75) (end 159.365 117.115) (width 0.4) (layer F.Cu) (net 13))
 (segment (start 159.365 117.115) (end 159.365 115.1) (width 0.4) (layer F.Cu) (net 13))
 (segment (start 161.905 109.7) (end 161.905 108.105035) (width 0.6) (layer F.Cu) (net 8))
 (segment (start 161.905 108.105035) (end 163 107.010035) (width 0.6) (layer F.Cu) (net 8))
 (segment (start 163 99.5) (end 162.5 99.5) (width 0.6) (layer F.Cu) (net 8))
 (segment (start 163 107.010035) (end 163 99.5) (width 0.6) (layer F.Cu) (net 8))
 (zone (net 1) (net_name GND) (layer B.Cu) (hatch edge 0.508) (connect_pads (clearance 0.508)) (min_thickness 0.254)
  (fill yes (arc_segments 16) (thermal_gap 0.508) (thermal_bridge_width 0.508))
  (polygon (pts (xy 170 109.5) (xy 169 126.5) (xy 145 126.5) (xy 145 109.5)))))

